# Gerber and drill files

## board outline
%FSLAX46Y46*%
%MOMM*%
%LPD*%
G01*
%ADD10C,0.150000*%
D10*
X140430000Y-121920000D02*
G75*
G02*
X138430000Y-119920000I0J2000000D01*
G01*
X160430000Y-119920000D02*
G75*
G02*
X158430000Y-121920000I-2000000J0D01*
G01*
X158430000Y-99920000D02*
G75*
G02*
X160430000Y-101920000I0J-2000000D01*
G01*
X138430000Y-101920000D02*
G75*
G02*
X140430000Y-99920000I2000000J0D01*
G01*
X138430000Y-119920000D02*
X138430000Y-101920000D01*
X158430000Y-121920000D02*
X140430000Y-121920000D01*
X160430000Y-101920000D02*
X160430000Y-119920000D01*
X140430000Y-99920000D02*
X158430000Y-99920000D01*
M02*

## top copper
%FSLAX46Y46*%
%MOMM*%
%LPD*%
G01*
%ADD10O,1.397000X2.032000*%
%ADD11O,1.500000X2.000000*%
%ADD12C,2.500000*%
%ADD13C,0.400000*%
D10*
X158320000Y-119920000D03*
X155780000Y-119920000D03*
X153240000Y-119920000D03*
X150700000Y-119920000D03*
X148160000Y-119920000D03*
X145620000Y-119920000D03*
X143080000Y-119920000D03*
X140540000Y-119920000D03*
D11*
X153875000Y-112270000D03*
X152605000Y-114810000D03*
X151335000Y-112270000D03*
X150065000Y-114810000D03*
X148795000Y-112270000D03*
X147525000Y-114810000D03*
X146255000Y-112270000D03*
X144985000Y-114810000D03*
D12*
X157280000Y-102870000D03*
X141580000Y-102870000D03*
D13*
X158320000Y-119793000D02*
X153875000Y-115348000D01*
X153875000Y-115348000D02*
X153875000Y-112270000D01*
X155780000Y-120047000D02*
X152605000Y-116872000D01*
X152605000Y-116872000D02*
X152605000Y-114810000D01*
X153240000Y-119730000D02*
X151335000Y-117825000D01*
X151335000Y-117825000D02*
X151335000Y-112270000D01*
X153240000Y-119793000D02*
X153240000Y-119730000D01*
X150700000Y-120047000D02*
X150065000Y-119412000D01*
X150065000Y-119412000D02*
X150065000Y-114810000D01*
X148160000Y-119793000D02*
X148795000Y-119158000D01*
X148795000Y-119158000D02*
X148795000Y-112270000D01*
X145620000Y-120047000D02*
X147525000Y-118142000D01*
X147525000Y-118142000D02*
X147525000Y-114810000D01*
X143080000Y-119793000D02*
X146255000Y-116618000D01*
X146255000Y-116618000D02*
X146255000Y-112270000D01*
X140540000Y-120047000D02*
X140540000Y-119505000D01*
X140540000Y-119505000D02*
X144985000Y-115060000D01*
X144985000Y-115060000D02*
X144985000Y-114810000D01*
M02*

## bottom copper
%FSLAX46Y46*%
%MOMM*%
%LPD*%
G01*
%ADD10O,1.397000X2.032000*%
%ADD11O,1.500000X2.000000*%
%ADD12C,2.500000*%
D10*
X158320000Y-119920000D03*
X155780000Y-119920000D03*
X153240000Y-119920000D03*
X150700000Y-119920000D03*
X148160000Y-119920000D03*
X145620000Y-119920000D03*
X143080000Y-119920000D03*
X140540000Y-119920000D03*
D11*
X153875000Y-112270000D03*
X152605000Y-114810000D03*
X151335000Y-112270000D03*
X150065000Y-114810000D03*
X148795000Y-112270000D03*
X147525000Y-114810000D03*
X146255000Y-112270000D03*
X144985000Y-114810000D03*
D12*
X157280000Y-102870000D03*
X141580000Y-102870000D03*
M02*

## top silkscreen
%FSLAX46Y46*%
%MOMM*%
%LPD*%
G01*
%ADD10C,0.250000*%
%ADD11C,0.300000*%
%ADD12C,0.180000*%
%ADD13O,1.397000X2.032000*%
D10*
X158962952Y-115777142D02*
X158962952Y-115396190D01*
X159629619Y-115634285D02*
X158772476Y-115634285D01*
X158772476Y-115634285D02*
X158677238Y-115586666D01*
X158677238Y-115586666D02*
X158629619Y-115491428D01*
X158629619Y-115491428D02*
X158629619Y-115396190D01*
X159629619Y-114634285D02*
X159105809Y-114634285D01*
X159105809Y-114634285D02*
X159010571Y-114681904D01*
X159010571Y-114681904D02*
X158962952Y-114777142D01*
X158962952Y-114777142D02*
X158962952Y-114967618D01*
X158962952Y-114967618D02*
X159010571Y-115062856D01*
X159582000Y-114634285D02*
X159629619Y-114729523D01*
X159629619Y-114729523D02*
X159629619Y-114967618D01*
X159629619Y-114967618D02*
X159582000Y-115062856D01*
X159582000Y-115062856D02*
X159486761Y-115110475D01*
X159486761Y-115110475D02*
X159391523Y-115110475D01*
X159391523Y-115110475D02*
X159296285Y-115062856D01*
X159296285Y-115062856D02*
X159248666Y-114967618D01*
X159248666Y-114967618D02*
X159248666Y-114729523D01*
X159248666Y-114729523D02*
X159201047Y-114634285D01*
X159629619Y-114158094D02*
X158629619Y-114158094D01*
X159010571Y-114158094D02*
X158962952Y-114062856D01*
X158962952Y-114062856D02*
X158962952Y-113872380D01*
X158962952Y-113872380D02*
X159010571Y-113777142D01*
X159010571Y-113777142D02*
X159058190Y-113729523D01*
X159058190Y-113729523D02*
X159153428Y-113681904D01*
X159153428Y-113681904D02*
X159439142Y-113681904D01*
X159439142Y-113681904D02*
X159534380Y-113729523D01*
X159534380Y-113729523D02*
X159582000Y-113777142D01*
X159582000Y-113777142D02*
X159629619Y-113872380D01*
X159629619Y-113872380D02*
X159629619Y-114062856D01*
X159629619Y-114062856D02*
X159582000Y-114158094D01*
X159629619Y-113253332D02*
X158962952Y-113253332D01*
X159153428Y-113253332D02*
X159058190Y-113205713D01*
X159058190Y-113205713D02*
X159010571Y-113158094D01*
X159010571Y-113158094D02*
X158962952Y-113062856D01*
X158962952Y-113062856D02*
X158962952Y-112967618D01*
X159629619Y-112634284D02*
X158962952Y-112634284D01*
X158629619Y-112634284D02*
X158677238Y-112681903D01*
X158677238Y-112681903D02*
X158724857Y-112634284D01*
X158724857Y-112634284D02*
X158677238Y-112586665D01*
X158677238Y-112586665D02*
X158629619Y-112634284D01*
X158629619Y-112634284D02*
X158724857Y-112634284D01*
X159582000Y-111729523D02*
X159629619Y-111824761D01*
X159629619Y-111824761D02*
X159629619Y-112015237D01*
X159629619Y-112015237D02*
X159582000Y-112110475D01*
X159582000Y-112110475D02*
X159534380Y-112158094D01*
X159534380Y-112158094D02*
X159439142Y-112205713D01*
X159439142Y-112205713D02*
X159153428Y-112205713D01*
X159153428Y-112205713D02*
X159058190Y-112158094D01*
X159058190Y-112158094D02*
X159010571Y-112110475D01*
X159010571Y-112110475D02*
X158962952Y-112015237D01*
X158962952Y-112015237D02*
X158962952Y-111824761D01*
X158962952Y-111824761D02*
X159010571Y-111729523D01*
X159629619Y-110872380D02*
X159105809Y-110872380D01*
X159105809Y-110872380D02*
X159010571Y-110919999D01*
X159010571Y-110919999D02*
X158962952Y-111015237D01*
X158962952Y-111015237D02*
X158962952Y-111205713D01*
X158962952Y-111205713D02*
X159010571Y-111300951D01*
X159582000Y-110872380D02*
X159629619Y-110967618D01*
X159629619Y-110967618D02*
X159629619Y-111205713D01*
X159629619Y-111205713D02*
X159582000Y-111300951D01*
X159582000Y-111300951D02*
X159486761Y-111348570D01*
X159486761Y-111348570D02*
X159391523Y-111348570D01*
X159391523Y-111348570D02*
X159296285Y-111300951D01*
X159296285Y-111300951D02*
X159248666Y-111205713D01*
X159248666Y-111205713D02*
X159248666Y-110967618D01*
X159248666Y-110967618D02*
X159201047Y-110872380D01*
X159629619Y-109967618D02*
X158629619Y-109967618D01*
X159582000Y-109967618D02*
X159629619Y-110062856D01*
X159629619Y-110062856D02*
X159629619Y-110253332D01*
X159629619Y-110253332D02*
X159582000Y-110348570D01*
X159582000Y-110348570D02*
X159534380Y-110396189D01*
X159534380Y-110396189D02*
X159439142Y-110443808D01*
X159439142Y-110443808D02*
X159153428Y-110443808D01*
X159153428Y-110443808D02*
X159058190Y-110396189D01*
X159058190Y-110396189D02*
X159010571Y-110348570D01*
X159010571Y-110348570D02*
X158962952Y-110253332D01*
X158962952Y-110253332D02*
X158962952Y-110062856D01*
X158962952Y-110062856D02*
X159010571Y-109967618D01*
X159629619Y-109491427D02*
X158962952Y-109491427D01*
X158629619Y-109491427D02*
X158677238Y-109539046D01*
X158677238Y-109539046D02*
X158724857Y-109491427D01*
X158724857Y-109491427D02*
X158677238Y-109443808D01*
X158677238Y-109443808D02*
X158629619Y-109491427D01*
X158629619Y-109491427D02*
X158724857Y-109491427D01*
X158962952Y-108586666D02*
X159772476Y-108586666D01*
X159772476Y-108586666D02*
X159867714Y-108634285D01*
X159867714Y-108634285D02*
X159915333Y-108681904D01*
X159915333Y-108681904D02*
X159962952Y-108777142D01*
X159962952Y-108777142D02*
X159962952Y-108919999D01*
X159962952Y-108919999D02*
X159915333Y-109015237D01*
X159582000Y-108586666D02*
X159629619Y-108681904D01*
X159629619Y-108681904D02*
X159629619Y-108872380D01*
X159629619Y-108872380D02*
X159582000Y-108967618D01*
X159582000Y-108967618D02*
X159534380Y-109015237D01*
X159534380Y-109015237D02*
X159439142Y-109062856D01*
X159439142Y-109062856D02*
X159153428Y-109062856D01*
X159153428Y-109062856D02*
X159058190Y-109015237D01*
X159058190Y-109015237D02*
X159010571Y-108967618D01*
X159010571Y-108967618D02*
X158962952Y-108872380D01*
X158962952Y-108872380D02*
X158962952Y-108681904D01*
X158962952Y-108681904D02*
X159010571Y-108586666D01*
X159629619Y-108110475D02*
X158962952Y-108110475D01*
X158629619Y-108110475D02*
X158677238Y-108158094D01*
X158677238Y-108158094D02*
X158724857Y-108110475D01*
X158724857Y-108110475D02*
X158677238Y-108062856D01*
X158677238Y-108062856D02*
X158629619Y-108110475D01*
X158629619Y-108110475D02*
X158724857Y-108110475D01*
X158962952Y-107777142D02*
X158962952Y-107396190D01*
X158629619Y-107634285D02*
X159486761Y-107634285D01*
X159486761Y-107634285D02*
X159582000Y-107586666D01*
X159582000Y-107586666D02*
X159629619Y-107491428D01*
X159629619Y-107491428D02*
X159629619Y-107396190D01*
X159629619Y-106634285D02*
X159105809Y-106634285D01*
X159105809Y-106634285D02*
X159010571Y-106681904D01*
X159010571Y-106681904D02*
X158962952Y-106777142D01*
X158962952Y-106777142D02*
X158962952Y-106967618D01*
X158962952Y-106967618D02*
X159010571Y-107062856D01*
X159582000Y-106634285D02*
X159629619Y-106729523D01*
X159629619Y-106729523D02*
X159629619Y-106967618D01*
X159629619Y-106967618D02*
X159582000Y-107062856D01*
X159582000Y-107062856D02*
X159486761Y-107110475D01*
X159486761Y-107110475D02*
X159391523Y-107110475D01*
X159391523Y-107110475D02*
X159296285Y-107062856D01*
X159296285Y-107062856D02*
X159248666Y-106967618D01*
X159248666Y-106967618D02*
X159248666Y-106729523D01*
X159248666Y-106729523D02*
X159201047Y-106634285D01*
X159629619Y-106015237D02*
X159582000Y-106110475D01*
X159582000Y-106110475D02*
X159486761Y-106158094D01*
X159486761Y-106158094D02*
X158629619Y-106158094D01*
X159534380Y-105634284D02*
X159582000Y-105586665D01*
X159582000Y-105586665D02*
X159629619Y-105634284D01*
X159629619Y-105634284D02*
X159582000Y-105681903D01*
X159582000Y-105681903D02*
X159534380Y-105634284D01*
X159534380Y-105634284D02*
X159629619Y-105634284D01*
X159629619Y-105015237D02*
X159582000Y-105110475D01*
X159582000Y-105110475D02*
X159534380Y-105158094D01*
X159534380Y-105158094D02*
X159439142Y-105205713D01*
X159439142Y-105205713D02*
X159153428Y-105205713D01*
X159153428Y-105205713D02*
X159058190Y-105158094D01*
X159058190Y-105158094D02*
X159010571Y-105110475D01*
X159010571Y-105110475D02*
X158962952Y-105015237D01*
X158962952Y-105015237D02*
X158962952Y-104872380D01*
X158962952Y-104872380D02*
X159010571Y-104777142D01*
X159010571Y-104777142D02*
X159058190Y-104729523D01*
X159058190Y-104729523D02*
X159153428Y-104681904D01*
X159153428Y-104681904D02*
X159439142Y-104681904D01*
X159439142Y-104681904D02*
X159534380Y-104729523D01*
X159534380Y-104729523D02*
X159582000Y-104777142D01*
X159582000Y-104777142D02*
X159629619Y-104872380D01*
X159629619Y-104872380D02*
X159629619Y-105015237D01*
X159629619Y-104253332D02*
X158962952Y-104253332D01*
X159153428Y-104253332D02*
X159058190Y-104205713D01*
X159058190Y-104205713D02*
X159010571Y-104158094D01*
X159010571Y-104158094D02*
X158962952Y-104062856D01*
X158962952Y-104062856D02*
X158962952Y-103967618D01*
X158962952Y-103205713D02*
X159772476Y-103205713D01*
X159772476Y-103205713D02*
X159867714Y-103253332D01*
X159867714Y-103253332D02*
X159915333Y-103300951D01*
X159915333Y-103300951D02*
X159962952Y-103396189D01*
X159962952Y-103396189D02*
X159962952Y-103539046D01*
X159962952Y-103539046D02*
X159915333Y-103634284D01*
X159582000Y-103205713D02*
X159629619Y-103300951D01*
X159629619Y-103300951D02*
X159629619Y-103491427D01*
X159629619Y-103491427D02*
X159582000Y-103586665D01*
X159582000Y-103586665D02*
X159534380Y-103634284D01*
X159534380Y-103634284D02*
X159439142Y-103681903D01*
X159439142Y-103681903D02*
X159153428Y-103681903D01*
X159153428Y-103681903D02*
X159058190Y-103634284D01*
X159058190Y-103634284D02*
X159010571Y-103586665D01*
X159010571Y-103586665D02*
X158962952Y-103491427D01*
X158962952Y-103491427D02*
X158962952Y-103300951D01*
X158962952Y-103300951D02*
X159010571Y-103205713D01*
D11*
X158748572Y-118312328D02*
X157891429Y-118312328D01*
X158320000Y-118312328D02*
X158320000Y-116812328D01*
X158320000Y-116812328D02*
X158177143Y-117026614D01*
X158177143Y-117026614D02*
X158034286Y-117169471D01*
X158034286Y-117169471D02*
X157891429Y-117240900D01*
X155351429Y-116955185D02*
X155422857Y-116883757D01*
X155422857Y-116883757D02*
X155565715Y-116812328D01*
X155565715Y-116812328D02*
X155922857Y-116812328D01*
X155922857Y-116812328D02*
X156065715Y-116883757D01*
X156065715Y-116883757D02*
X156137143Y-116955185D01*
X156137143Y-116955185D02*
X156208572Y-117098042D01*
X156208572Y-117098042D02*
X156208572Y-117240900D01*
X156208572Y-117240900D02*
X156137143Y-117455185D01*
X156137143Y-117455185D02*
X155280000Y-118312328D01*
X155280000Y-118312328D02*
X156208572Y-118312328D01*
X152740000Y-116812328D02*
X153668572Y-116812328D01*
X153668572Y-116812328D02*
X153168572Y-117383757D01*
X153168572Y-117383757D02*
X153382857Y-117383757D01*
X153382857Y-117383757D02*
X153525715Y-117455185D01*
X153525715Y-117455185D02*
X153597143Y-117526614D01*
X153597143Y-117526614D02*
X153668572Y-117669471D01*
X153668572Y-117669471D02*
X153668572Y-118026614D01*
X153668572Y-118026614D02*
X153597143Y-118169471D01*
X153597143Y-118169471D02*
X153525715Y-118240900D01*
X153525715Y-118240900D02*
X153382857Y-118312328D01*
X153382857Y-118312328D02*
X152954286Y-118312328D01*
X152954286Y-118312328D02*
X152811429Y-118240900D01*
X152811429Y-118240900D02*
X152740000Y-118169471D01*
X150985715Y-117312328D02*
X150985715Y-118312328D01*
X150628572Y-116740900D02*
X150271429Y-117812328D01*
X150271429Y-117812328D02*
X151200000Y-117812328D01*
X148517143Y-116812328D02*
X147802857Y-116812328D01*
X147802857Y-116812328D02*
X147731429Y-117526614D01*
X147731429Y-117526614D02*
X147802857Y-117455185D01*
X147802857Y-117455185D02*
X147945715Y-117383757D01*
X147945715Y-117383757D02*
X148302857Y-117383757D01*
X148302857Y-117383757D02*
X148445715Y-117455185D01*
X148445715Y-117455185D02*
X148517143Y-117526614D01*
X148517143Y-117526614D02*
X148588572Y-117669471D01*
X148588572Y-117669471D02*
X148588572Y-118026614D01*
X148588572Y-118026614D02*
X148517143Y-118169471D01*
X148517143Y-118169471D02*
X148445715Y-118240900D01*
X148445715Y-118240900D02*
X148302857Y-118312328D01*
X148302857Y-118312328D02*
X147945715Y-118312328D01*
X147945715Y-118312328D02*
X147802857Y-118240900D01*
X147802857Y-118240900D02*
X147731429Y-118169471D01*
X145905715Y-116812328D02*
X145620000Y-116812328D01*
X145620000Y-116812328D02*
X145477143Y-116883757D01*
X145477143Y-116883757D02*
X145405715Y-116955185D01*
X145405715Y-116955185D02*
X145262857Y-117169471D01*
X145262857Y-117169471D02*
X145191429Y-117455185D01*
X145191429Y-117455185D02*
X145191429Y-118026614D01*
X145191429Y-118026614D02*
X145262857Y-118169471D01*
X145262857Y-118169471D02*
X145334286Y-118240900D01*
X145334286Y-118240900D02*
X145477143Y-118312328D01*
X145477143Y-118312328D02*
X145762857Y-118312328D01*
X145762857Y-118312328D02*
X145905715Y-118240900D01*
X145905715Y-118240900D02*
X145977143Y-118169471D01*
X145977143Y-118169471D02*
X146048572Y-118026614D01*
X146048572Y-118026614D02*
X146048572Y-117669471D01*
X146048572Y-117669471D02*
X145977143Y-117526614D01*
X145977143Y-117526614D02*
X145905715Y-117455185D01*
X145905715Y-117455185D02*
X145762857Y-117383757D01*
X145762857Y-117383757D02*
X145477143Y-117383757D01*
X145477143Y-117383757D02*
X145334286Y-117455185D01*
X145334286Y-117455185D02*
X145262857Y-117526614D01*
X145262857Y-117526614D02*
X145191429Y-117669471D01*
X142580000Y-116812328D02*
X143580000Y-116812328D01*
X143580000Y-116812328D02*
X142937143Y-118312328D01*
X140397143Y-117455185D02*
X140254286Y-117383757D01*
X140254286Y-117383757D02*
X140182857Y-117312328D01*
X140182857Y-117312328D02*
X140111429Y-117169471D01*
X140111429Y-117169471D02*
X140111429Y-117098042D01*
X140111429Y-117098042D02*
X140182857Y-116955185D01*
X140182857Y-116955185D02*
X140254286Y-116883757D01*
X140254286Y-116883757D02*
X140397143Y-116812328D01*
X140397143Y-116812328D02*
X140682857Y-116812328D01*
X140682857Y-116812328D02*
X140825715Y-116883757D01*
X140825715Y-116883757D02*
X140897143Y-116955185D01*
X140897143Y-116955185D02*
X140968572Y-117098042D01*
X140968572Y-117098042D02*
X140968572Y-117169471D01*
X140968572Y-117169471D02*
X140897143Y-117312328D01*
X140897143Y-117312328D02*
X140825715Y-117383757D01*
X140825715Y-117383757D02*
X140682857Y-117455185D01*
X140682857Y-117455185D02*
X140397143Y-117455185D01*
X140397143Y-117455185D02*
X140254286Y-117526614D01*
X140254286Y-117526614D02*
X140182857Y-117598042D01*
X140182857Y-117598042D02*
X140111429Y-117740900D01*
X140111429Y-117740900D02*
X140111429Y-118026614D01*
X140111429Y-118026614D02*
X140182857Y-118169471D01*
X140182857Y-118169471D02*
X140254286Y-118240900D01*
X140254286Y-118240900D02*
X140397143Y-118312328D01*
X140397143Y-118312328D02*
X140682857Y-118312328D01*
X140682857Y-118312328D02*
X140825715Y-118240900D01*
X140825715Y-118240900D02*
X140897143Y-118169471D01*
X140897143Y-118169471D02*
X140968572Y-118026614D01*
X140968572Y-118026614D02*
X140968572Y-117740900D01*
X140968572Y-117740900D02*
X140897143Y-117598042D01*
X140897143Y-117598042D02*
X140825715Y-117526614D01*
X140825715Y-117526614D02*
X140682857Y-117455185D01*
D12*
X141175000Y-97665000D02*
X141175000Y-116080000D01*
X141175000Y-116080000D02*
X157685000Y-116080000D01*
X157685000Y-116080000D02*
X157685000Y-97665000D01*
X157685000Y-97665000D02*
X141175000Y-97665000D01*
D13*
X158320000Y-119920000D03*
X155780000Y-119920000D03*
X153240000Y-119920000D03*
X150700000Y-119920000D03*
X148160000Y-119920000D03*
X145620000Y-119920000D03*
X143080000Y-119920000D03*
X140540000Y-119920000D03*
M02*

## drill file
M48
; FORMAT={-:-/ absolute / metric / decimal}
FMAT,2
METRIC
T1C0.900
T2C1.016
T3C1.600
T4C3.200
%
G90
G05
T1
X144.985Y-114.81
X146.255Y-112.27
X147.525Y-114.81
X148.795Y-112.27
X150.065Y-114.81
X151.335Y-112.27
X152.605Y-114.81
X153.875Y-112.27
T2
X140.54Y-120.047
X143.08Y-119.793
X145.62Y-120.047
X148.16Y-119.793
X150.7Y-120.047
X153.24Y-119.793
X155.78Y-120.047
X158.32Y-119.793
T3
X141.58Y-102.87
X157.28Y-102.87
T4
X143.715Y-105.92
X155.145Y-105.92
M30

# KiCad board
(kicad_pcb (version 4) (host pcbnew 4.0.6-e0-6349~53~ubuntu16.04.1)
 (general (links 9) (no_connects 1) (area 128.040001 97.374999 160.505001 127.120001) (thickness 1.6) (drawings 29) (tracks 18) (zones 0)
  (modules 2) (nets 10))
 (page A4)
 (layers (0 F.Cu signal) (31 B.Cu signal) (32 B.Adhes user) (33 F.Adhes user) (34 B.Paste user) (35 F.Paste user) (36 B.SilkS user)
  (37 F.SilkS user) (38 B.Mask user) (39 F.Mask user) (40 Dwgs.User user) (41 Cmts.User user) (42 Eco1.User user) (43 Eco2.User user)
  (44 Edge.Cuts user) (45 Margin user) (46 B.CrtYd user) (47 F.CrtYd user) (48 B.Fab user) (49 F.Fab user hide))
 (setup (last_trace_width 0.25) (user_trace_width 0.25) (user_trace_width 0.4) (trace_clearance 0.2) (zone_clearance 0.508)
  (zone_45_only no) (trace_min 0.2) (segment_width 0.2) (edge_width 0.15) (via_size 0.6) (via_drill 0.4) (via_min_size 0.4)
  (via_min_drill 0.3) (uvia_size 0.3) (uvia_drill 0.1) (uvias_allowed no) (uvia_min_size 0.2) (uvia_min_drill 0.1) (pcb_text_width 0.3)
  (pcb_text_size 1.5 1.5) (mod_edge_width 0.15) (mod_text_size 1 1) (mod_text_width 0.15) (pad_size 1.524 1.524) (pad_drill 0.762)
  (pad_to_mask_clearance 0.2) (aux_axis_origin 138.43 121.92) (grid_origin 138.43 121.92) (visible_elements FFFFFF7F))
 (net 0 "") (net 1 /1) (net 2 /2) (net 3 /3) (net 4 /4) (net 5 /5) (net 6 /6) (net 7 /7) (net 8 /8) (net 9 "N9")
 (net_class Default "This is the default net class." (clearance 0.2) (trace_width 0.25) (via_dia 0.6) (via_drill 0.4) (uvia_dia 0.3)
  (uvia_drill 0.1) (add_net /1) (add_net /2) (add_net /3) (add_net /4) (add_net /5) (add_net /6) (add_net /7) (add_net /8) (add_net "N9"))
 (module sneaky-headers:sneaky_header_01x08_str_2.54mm (layer F.Cu) (at 149.43 119.92 180)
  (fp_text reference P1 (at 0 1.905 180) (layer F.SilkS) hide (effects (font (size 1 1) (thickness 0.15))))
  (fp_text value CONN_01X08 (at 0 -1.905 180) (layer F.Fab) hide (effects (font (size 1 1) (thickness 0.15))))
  (pad 1 thru_hole oval (at -8.89 0.127 180) (size 1.397 2.032) (drill 1.016 (offset 0 -0.127)) (layers *.Cu *.Mask F.SilkS) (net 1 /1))
  (pad 2 thru_hole oval (at -6.35 -0.127 180) (size 1.397 2.032) (drill 1.016 (offset 0 0.127)) (layers *.Cu *.Mask F.SilkS) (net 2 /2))
  (pad 3 thru_hole oval (at -3.81 0.127 180) (size 1.397 2.032) (drill 1.016 (offset 0 -0.127)) (layers *.Cu *.Mask F.SilkS) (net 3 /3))
  (pad 4 thru_hole oval (at -1.27 -0.127 180) (size 1.397 2.032) (drill 1.016 (offset 0 0.127)) (layers *.Cu *.Mask F.SilkS) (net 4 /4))
  (pad 5 thru_hole oval (at 1.27 0.127 180) (size 1.397 2.032) (drill 1.016 (offset 0 -0.127)) (layers *.Cu *.Mask F.SilkS) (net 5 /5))
  (pad 6 thru_hole oval (at 3.81 -0.127 180) (size 1.397 2.032) (drill 1.016 (offset 0 0.127)) (layers *.Cu *.Mask F.SilkS) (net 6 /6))
  (pad 7 thru_hole oval (at 6.35 0.127 180) (size 1.397 2.032) (drill 1.016 (offset 0 -0.127)) (layers *.Cu *.Mask F.SilkS) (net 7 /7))
  (pad 8 thru_hole oval (at 8.89 -0.127 180) (size 1.397 2.032) (drill 1.016 (offset 0 0.127)) (layers *.Cu *.Mask F.SilkS) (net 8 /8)))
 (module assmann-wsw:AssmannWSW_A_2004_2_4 (layer F.Cu) (at 149.43 105.92 180)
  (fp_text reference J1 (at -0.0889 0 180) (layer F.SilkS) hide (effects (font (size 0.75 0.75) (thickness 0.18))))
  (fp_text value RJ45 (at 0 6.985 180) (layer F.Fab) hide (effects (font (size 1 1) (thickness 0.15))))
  (fp_line (start 8.255 8.255) (end 8.255 -10.16) (layer F.SilkS) (width 0.18))
  (fp_line (start 8.255 -10.16) (end -8.255 -10.16) (layer F.SilkS) (width 0.18))
  (fp_line (start -8.255 -10.16) (end -8.255 8.255) (layer F.SilkS) (width 0.18))
  (fp_line (start -8.255 8.255) (end 8.255 8.255) (layer F.SilkS) (width 0.18))
  (pad "" np_thru_hole circle (at -5.715 0 180) (size 3.2 3.2) (drill 3.2) (layers *.Cu *.Mask))
  (pad "" np_thru_hole circle (at 5.715 0 180) (size 3.2 3.2) (drill 3.2) (layers *.Cu *.Mask))
  (pad 1 thru_hole oval (at -4.445 -6.35 180) (size 1.5 2) (drill 0.9) (layers *.Cu *.Mask) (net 1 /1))
  (pad 2 thru_hole oval (at -3.175 -8.89 180) (size 1.5 2) (drill 0.9) (layers *.Cu *.Mask) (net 2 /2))
  (pad 3 thru_hole oval (at -1.905 -6.35 180) (size 1.5 2) (drill 0.9) (layers *.Cu *.Mask) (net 3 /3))
  (pad 4 thru_hole oval (at -0.635 -8.89 180) (size 1.5 2) (drill 0.9) (layers *.Cu *.Mask) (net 4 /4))
  (pad 5 thru_hole oval (at 0.635 -6.35 180) (size 1.5 2) (drill 0.9) (layers *.Cu *.Mask) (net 5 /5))
  (pad 6 thru_hole oval (at 1.905 -8.89 180) (size 1.5 2) (drill 0.9) (layers *.Cu *.Mask) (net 6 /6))
  (pad 7 thru_hole oval (at 3.175 -6.35 180) (size 1.5 2) (drill 0.9) (layers *.Cu *.Mask) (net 7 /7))
  (pad 8 thru_hole oval (at 4.445 -8.89 180) (size 1.5 2) (drill 0.9) (layers *.Cu *.Mask) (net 8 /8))
  (pad 9 thru_hole circle (at -7.85 3.05 180) (size 2.5 2.5) (drill 1.6) (layers *.Cu *.Mask) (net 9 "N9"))
  (pad 9 thru_hole circle (at 7.85 3.05 180) (size 2.5 2.5) (drill 1.6) (layers *.Cu *.Mask) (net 9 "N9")))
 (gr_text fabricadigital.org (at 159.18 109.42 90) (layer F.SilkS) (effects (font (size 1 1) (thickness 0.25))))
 (gr_arc (start 140.43 119.92) (end 140.43 121.92) (angle 90) (layer Edge.Cuts) (width 0.15))
 (gr_arc (start 158.43 119.92) (end 160.43 119.92) (angle 90) (layer Edge.Cuts) (width 0.15))
 (gr_arc (start 158.43 101.92) (end 158.43 99.92) (angle 90) (layer Edge.Cuts) (width 0.15))
 (gr_arc (start 140.43 101.92) (end 138.43 101.92) (angle 90) (layer Edge.Cuts) (width 0.15))
 (gr_line (start 138.43 119.92) (end 138.43 101.92) (layer Edge.Cuts) (width 0.15))
 (gr_line (start 158.43 121.92) (end 140.43 121.92) (layer Edge.Cuts) (width 0.15))
 (gr_line (start 160.43 101.92) (end 160.43 119.92) (layer Edge.Cuts) (width 0.15))
 (gr_line (start 140.43 99.92) (end 158.43 99.92) (layer Edge.Cuts) (width 0.15))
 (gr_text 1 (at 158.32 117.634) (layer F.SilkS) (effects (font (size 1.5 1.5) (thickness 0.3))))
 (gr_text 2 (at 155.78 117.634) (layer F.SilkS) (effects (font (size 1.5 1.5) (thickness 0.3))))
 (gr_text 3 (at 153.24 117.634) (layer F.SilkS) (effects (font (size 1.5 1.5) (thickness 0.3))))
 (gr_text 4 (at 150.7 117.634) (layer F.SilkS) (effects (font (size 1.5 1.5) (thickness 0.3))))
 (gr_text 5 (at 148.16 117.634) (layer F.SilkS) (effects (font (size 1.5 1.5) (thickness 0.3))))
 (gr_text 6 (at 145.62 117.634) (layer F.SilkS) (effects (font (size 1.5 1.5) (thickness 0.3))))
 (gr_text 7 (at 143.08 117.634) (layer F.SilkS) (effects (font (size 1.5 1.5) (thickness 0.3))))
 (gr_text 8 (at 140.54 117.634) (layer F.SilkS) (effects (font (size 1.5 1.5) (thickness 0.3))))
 (segment (start 158.32 119.793) (end 153.875 115.348) (width 0.4) (layer F.Cu) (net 1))
 (segment (start 153.875 115.348) (end 153.875 112.27) (width 0.4) (layer F.Cu) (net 1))
 (segment (start 155.78 120.047) (end 152.605 116.872) (width 0.4) (layer F.Cu) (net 2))
 (segment (start 152.605 116.872) (end 152.605 114.81) (width 0.4) (layer F.Cu) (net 2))
 (segment (start 153.24 119.73) (end 151.335 117.825) (width 0.4) (layer F.Cu) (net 3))
 (segment (start 151.335 117.825) (end 151.335 112.27) (width 0.4) (layer F.Cu) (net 3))
 (segment (start 153.24 119.793) (end 153.24 119.73) (width 0.4) (layer F.Cu) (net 3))
 (segment (start 150.7 120.047) (end 150.065 119.412) (width 0.4) (layer F.Cu) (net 4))
 (segment (start 150.065 119.412) (end 150.065 114.81) (width 0.4) (layer F.Cu) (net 4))
 (segment (start 148.16 119.793) (end 148.795 119.158) (width 0.4) (layer F.Cu) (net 5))
 (segment (start 148.795 119.158) (end 148.795 112.27) (width 0.4) (layer F.Cu) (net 5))
 (segment (start 145.62 120.047) (end 147.525 118.142) (width 0.4) (layer F.Cu) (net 6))
 (segment (start 147.525 118.142) (end 147.525 114.81) (width 0.4) (layer F.Cu) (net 6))
 (segment (start 143.08 119.793) (end 146.255 116.618) (width 0.4) (layer F.Cu) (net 7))
 (segment (start 146.255 116.618) (end 146.255 112.27) (width 0.4) (layer F.Cu) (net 7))
 (segment (start 140.54 120.047) (end 140.54 119.505) (width 0.4) (layer F.Cu) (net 8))
 (segment (start 140.54 119.505) (end 144.985 115.06) (width 0.4) (layer F.Cu) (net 8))
 (segment (start 144.985 115.06) (end 144.985 114.81) (width 0.4) (layer F.Cu) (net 8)))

